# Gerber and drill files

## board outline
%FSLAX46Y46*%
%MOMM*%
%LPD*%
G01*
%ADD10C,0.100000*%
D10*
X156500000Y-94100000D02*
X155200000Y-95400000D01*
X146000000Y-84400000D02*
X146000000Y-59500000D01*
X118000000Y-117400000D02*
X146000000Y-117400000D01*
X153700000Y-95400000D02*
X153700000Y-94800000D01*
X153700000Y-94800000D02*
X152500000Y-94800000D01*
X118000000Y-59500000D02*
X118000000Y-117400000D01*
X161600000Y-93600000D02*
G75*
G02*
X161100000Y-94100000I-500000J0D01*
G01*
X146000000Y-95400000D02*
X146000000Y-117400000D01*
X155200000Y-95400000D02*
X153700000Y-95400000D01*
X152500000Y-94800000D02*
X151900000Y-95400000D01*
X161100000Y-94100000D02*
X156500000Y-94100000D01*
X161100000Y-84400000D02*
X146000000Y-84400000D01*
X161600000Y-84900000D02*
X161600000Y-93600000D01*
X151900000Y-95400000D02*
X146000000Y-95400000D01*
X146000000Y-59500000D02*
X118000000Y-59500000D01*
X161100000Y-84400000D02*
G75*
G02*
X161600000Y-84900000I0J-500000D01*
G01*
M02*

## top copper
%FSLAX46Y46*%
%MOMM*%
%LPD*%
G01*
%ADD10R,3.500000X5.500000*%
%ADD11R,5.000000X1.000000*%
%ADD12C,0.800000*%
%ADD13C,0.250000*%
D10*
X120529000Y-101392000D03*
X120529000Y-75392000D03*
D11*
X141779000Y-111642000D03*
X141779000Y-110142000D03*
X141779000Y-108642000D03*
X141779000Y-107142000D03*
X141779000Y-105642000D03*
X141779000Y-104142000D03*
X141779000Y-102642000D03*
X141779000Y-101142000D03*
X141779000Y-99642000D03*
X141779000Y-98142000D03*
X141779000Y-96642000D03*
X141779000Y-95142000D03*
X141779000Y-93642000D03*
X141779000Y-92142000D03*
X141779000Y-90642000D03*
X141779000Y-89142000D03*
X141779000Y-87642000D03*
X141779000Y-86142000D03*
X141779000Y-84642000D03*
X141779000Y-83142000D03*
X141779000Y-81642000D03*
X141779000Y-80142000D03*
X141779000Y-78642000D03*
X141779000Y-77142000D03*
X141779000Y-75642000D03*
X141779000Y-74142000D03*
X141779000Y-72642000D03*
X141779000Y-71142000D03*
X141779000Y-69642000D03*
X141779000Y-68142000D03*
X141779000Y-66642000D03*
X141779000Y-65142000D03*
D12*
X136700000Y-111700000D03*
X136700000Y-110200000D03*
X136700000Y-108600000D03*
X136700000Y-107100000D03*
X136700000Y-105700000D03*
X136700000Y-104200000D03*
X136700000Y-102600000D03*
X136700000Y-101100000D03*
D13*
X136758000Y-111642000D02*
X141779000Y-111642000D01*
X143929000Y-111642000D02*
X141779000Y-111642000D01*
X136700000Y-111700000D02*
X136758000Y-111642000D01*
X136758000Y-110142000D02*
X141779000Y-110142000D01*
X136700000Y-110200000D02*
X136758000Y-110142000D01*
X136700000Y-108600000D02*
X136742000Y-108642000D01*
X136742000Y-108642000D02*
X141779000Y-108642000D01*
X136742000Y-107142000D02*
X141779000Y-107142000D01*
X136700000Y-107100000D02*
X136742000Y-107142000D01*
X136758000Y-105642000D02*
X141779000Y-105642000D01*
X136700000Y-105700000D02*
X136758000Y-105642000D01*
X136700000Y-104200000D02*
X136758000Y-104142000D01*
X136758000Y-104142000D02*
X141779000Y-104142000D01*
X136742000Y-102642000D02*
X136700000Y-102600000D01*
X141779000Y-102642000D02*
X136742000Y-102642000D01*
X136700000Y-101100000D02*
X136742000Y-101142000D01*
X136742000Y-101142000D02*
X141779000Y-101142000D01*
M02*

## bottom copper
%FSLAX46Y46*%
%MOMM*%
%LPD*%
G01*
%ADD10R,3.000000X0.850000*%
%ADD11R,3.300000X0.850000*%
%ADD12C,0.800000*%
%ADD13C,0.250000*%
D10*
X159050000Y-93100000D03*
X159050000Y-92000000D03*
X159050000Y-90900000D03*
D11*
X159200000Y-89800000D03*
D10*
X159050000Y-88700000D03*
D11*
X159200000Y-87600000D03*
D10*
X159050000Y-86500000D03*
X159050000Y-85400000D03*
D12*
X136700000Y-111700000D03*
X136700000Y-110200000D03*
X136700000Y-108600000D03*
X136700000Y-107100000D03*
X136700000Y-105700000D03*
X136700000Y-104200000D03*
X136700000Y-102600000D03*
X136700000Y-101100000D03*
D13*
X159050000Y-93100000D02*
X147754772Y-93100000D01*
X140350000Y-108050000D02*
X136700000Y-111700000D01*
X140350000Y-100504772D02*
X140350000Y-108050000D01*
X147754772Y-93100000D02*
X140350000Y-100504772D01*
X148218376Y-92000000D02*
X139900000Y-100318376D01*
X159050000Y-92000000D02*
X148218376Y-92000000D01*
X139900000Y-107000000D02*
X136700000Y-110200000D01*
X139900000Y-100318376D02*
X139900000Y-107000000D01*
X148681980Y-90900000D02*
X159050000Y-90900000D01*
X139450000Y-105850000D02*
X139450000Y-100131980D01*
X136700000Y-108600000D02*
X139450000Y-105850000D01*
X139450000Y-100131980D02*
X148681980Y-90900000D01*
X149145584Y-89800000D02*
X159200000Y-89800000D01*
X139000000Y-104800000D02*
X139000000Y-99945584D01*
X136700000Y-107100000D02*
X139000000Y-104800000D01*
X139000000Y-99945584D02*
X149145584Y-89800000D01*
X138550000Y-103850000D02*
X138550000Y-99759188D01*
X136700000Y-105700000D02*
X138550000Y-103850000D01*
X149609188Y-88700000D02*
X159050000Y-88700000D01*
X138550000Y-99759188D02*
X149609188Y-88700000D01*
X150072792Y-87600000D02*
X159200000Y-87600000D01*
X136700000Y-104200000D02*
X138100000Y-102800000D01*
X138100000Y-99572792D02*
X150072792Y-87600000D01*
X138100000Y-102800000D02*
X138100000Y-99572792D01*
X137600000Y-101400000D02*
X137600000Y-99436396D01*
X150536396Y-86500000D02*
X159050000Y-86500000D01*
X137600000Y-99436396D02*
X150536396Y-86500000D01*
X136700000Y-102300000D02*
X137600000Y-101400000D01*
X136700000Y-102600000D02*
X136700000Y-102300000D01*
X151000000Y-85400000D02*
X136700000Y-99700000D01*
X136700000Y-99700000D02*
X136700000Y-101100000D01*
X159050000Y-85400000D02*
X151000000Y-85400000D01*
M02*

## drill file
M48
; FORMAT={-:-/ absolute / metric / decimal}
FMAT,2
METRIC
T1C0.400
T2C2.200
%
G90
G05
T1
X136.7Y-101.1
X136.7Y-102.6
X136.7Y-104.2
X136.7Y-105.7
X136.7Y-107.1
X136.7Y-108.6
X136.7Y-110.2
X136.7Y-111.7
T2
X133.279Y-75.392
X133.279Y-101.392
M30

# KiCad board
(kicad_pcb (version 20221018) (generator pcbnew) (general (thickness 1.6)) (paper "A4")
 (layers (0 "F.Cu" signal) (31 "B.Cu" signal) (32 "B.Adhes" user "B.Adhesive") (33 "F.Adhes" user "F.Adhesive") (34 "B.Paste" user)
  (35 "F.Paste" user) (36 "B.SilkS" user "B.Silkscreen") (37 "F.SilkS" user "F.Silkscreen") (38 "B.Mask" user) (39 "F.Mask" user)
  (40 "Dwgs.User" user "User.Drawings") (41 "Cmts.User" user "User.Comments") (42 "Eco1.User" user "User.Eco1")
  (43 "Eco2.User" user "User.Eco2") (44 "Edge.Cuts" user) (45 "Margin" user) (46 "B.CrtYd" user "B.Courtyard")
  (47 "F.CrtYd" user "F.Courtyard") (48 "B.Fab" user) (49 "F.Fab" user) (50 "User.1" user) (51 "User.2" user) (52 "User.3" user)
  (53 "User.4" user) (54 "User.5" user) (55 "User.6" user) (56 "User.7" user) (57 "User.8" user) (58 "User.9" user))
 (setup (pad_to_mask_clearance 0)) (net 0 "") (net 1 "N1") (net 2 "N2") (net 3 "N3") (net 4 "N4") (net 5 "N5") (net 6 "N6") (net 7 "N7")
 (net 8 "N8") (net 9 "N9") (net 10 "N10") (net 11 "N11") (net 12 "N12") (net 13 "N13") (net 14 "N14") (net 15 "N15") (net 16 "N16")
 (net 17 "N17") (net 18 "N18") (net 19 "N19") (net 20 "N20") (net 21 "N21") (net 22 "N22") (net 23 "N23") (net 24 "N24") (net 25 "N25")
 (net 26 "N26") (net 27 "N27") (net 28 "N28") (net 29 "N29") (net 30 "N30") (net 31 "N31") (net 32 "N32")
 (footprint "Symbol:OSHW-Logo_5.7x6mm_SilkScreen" (layer "F.Cu") (at 155 89.2 -90)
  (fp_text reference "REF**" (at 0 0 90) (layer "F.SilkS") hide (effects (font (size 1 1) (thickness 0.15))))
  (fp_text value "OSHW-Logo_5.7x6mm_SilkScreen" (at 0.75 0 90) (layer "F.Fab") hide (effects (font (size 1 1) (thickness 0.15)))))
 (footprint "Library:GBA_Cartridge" (layer "F.Cu") (at 136.779 88.392 180)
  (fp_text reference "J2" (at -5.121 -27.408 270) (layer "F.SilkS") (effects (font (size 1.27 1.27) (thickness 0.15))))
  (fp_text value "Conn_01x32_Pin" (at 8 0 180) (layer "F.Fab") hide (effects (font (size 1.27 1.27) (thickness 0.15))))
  (pad "" np_thru_hole circle (at 3.5 -13 180) (size 2.2 2.2) (drill 2.2) (layers "*.Cu" "*.Mask"))
  (pad "" np_thru_hole circle (at 3.5 13 180) (size 2.2 2.2) (drill 2.2) (layers "*.Cu" "*.Mask"))
  (pad "" smd rect (at 16.25 -13 90) (size 5.5 3.5) (layers "F.Cu" "F.Paste" "F.Mask"))
  (pad "" smd rect (at 16.25 13 90) (size 5.5 3.5) (layers "F.Cu" "F.Paste" "F.Mask"))
  (pad "1" smd rect (at -5 -23.25) (size 5 1) (layers "F.Cu" "F.Paste" "F.Mask") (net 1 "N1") (solder_mask_margin 0.0508))
  (pad "2" smd rect (at -5 -21.75) (size 5 1) (layers "F.Cu" "F.Paste" "F.Mask") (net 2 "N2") (solder_mask_margin 0.0508))
  (pad "3" smd rect (at -5 -20.25) (size 5 1) (layers "F.Cu" "F.Paste" "F.Mask") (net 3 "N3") (solder_mask_margin 0.0508))
  (pad "4" smd rect (at -5 -18.75) (size 5 1) (layers "F.Cu" "F.Paste" "F.Mask") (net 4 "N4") (solder_mask_margin 0.0508))
  (pad "5" smd rect (at -5 -17.25) (size 5 1) (layers "F.Cu" "F.Paste" "F.Mask") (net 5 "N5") (solder_mask_margin 0.0508))
  (pad "6" smd rect (at -5 -15.75) (size 5 1) (layers "F.Cu" "F.Paste" "F.Mask") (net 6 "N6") (solder_mask_margin 0.0508))
  (pad "7" smd rect (at -5 -14.25) (size 5 1) (layers "F.Cu" "F.Paste" "F.Mask") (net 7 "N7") (solder_mask_margin 0.0508))
  (pad "8" smd rect (at -5 -12.75) (size 5 1) (layers "F.Cu" "F.Paste" "F.Mask") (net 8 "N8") (solder_mask_margin 0.0508))
  (pad "9" smd rect (at -5 -11.25) (size 5 1) (layers "F.Cu" "F.Paste" "F.Mask") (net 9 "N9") (solder_mask_margin 0.0508))
  (pad "10" smd rect (at -5 -9.75) (size 5 1) (layers "F.Cu" "F.Paste" "F.Mask") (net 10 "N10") (solder_mask_margin 0.0508))
  (pad "11" smd rect (at -5 -8.25) (size 5 1) (layers "F.Cu" "F.Paste" "F.Mask") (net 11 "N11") (solder_mask_margin 0.0508))
  (pad "12" smd rect (at -5 -6.75) (size 5 1) (layers "F.Cu" "F.Paste" "F.Mask") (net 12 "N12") (solder_mask_margin 0.0508))
  (pad "13" smd rect (at -5 -5.25) (size 5 1) (layers "F.Cu" "F.Paste" "F.Mask") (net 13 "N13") (solder_mask_margin 0.0508))
  (pad "14" smd rect (at -5 -3.75) (size 5 1) (layers "F.Cu" "F.Paste" "F.Mask") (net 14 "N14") (solder_mask_margin 0.0508))
  (pad "15" smd rect (at -5 -2.25) (size 5 1) (layers "F.Cu" "F.Paste" "F.Mask") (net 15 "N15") (solder_mask_margin 0.0508))
  (pad "16" smd rect (at -5 -0.75) (size 5 1) (layers "F.Cu" "F.Paste" "F.Mask") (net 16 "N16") (solder_mask_margin 0.0508))
  (pad "17" smd rect (at -5 0.75) (size 5 1) (layers "F.Cu" "F.Paste" "F.Mask") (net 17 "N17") (solder_mask_margin 0.0508))
  (pad "18" smd rect (at -5 2.25) (size 5 1) (layers "F.Cu" "F.Paste" "F.Mask") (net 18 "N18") (solder_mask_margin 0.0508))
  (pad "19" smd rect (at -5 3.75) (size 5 1) (layers "F.Cu" "F.Paste" "F.Mask") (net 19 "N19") (solder_mask_margin 0.0508))
  (pad "20" smd rect (at -5 5.25) (size 5 1) (layers "F.Cu" "F.Paste" "F.Mask") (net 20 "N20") (solder_mask_margin 0.0508))
  (pad "21" smd rect (at -5 6.75) (size 5 1) (layers "F.Cu" "F.Paste" "F.Mask") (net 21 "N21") (solder_mask_margin 0.0508))
  (pad "22" smd rect (at -5 8.25) (size 5 1) (layers "F.Cu" "F.Paste" "F.Mask") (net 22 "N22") (solder_mask_margin 0.0508))
  (pad "23" smd rect (at -5 9.75) (size 5 1) (layers "F.Cu" "F.Paste" "F.Mask") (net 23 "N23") (solder_mask_margin 0.0508))
  (pad "24" smd rect (at -5 11.25) (size 5 1) (layers "F.Cu" "F.Paste" "F.Mask") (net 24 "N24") (solder_mask_margin 0.0508))
  (pad "25" smd rect (at -5 12.75) (size 5 1) (layers "F.Cu" "F.Paste" "F.Mask") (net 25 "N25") (solder_mask_margin 0.0508))
  (pad "26" smd rect (at -5 14.25) (size 5 1) (layers "F.Cu" "F.Paste" "F.Mask") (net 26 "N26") (solder_mask_margin 0.0508))
  (pad "27" smd rect (at -5 15.75) (size 5 1) (layers "F.Cu" "F.Paste" "F.Mask") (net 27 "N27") (solder_mask_margin 0.0508))
  (pad "28" smd rect (at -5 17.25) (size 5 1) (layers "F.Cu" "F.Paste" "F.Mask") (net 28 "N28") (solder_mask_margin 0.0508))
  (pad "29" smd rect (at -5 18.75) (size 5 1) (layers "F.Cu" "F.Paste" "F.Mask") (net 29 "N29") (solder_mask_margin 0.0508))
  (pad "30" smd rect (at -5 20.25) (size 5 1) (layers "F.Cu" "F.Paste" "F.Mask") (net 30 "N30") (solder_mask_margin 0.0508))
  (pad "31" smd rect (at -5 21.75) (size 5 1) (layers "F.Cu" "F.Paste" "F.Mask") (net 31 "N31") (solder_mask_margin 0.0508))
  (pad "32" smd rect (at -5 23.25) (size 5 1) (layers "F.Cu" "F.Paste" "F.Mask") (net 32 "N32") (solder_mask_margin 0.0508)))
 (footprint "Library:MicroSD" (layer "B.Cu") (at 161.6 84.4 90)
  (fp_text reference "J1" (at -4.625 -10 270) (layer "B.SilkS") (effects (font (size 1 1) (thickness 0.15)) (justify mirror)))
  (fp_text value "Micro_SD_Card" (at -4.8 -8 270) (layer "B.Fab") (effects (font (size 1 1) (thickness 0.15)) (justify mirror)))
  (pad "1" connect rect (at -8.7 -2.55 270) (size 0.85 3) (layers "B.Cu" "B.Mask") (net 1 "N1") (solder_mask_margin 0.05))
  (pad "2" connect rect (at -7.6 -2.55 270) (size 0.85 3) (layers "B.Cu" "B.Mask") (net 2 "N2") (solder_mask_margin 0.05))
  (pad "3" connect rect (at -6.5 -2.55 270) (size 0.85 3) (layers "B.Cu" "B.Mask") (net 3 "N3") (solder_mask_margin 0.05))
  (pad "4" connect rect (at -5.4 -2.4 270) (size 0.85 3.3) (layers "B.Cu" "B.Mask") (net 4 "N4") (solder_mask_margin 0.05))
  (pad "5" connect rect (at -4.3 -2.55 270) (size 0.85 3) (layers "B.Cu" "B.Mask") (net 5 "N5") (solder_mask_margin 0.05))
  (pad "6" connect rect (at -3.2 -2.4 270) (size 0.85 3.3) (layers "B.Cu" "B.Mask") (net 6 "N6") (solder_mask_margin 0.05))
  (pad "7" connect rect (at -2.1 -2.55 270) (size 0.85 3) (layers "B.Cu" "B.Mask") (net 7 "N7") (solder_mask_margin 0.05))
  (pad "8" connect rect (at -1 -2.55 270) (size 0.85 3) (layers "B.Cu" "B.Mask") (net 8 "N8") (solder_mask_margin 0.05)))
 (gr_line (start 156.5 94.1) (end 155.2 95.4) (stroke (width 0.1) (type default)) (layer "Edge.Cuts"))
 (gr_line (start 146 84.4) (end 146 59.5) (stroke (width 0.1) (type default)) (layer "Edge.Cuts"))
 (gr_line (start 118 117.4) (end 146 117.4) (stroke (width 0.1) (type default)) (layer "Edge.Cuts"))
 (gr_line (start 153.7 95.4) (end 153.7 94.8) (stroke (width 0.1) (type default)) (layer "Edge.Cuts"))
 (gr_line (start 153.7 94.8) (end 152.5 94.8) (stroke (width 0.1) (type default)) (layer "Edge.Cuts"))
 (gr_line (start 118 59.5) (end 118 117.4) (stroke (width 0.1) (type default)) (layer "Edge.Cuts"))
 (gr_arc (start 161.6 93.6) (mid 161.453553 93.953553) (end 161.1 94.1) (stroke (width 0.1) (type default)) (layer "Edge.Cuts"))
 (gr_line (start 146 95.4) (end 146 117.4) (stroke (width 0.1) (type default)) (layer "Edge.Cuts"))
 (gr_line (start 155.2 95.4) (end 153.7 95.4) (stroke (width 0.1) (type default)) (layer "Edge.Cuts"))
 (gr_line (start 152.5 94.8) (end 151.9 95.4) (stroke (width 0.1) (type default)) (layer "Edge.Cuts"))
 (gr_line (start 161.1 94.1) (end 156.5 94.1) (stroke (width 0.1) (type default)) (layer "Edge.Cuts"))
 (gr_line (start 161.1 84.4) (end 146 84.4) (stroke (width 0.1) (type default)) (layer "Edge.Cuts"))
 (gr_line (start 161.6 84.9) (end 161.6 93.6) (stroke (width 0.1) (type default)) (layer "Edge.Cuts"))
 (gr_line (start 151.9 95.4) (end 146 95.4) (stroke (width 0.1) (type default)) (layer "Edge.Cuts"))
 (gr_line (start 146 59.5) (end 118 59.5) (stroke (width 0.1) (type default)) (layer "Edge.Cuts"))
 (gr_arc (start 161.1 84.4) (mid 161.453553 84.546447) (end 161.6 84.9) (stroke (width 0.1) (type default)) (layer "Edge.Cuts"))
 (segment (start 136.758 111.642) (end 141.779 111.642) (width 0.25) (layer "F.Cu") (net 1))
 (segment (start 143.929 111.642) (end 141.779 111.642) (width 0.25) (layer "F.Cu") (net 1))
 (segment (start 136.7 111.7) (end 136.758 111.642) (width 0.25) (layer "F.Cu") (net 1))
 (via (at 136.7 111.7) (size 0.8) (drill 0.4) (layers "F.Cu" "B.Cu") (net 1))
 (segment (start 159.05 93.1) (end 147.754772 93.1) (width 0.25) (layer "B.Cu") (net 1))
 (segment (start 140.35 108.05) (end 136.7 111.7) (width 0.25) (layer "B.Cu") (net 1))
 (segment (start 140.35 100.504772) (end 140.35 108.05) (width 0.25) (layer "B.Cu") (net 1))
 (segment (start 147.754772 93.1) (end 140.35 100.504772) (width 0.25) (layer "B.Cu") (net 1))
 (segment (start 136.758 110.142) (end 141.779 110.142) (width 0.25) (layer "F.Cu") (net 2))
 (segment (start 136.7 110.2) (end 136.758 110.142) (width 0.25) (layer "F.Cu") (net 2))
 (via (at 136.7 110.2) (size 0.8) (drill 0.4) (layers "F.Cu" "B.Cu") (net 2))
 (segment (start 148.218376 92) (end 139.9 100.318376) (width 0.25) (layer "B.Cu") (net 2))
 (segment (start 159.05 92) (end 148.218376 92) (width 0.25) (layer "B.Cu") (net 2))
 (segment (start 139.9 107) (end 136.7 110.2) (width 0.25) (layer "B.Cu") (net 2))
 (segment (start 139.9 100.318376) (end 139.9 107) (width 0.25) (layer "B.Cu") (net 2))
 (segment (start 136.7 108.6) (end 136.742 108.642) (width 0.25) (layer "F.Cu") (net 3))
 (segment (start 136.742 108.642) (end 141.779 108.642) (width 0.25) (layer "F.Cu") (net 3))
 (via (at 136.7 108.6) (size 0.8) (drill 0.4) (layers "F.Cu" "B.Cu") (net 3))
 (segment (start 148.68198 90.9) (end 159.05 90.9) (width 0.25) (layer "B.Cu") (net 3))
 (segment (start 139.45 105.85) (end 139.45 100.13198) (width 0.25) (layer "B.Cu") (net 3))
 (segment (start 136.7 108.6) (end 139.45 105.85) (width 0.25) (layer "B.Cu") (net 3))
 (segment (start 139.45 100.13198) (end 148.68198 90.9) (width 0.25) (layer "B.Cu") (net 3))
 (segment (start 136.742 107.142) (end 141.779 107.142) (width 0.25) (layer "F.Cu") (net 4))
 (segment (start 136.7 107.1) (end 136.742 107.142) (width 0.25) (layer "F.Cu") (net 4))
 (via (at 136.7 107.1) (size 0.8) (drill 0.4) (layers "F.Cu" "B.Cu") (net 4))
 (segment (start 149.145584 89.8) (end 159.2 89.8) (width 0.25) (layer "B.Cu") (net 4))
 (segment (start 139 104.8) (end 139 99.945584) (width 0.25) (layer "B.Cu") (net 4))
 (segment (start 136.7 107.1) (end 139 104.8) (width 0.25) (layer "B.Cu") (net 4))
 (segment (start 139 99.945584) (end 149.145584 89.8) (width 0.25) (layer "B.Cu") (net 4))
 (segment (start 136.758 105.642) (end 141.779 105.642) (width 0.25) (layer "F.Cu") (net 5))
 (segment (start 136.7 105.7) (end 136.758 105.642) (width 0.25) (layer "F.Cu") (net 5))
 (via (at 136.7 105.7) (size 0.8) (drill 0.4) (layers "F.Cu" "B.Cu") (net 5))
 (segment (start 138.55 103.85) (end 138.55 99.759188) (width 0.25) (layer "B.Cu") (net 5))
 (segment (start 136.7 105.7) (end 138.55 103.85) (width 0.25) (layer "B.Cu") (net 5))
 (segment (start 149.609188 88.7) (end 159.05 88.7) (width 0.25) (layer "B.Cu") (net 5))
 (segment (start 138.55 99.759188) (end 149.609188 88.7) (width 0.25) (layer "B.Cu") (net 5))
 (segment (start 136.7 104.2) (end 136.758 104.142) (width 0.25) (layer "F.Cu") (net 6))
 (segment (start 136.758 104.142) (end 141.779 104.142) (width 0.25) (layer "F.Cu") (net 6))
 (via (at 136.7 104.2) (size 0.8) (drill 0.4) (layers "F.Cu" "B.Cu") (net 6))
 (segment (start 150.072792 87.6) (end 159.2 87.6) (width 0.25) (layer "B.Cu") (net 6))
 (segment (start 136.7 104.2) (end 138.1 102.8) (width 0.25) (layer "B.Cu") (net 6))
 (segment (start 138.1 99.572792) (end 150.072792 87.6) (width 0.25) (layer "B.Cu") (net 6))
 (segment (start 138.1 102.8) (end 138.1 99.572792) (width 0.25) (layer "B.Cu") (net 6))
 (segment (start 136.742 102.642) (end 136.7 102.6) (width 0.25) (layer "F.Cu") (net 7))
 (segment (start 141.779 102.642) (end 136.742 102.642) (width 0.25) (layer "F.Cu") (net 7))
 (via (at 136.7 102.6) (size 0.8) (drill 0.4) (layers "F.Cu" "B.Cu") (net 7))
 (segment (start 137.6 101.4) (end 137.6 99.436396) (width 0.25) (layer "B.Cu") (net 7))
 (segment (start 150.536396 86.5) (end 159.05 86.5) (width 0.25) (layer "B.Cu") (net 7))
 (segment (start 137.6 99.436396) (end 150.536396 86.5) (width 0.25) (layer "B.Cu") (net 7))
 (segment (start 136.7 102.3) (end 137.6 101.4) (width 0.25) (layer "B.Cu") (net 7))
 (segment (start 136.7 102.6) (end 136.7 102.3) (width 0.25) (layer "B.Cu") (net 7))
 (segment (start 136.7 101.1) (end 136.742 101.142) (width 0.25) (layer "F.Cu") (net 8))
 (segment (start 136.742 101.142) (end 141.779 101.142) (width 0.25) (layer "F.Cu") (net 8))
 (via (at 136.7 101.1) (size 0.8) (drill 0.4) (layers "F.Cu" "B.Cu") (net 8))
 (segment (start 151 85.4) (end 136.7 99.7) (width 0.25) (layer "B.Cu") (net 8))
 (segment (start 136.7 99.7) (end 136.7 101.1) (width 0.25) (layer "B.Cu") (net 8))
 (segment (start 159.05 85.4) (end 151 85.4) (width 0.25) (layer "B.Cu") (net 8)))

